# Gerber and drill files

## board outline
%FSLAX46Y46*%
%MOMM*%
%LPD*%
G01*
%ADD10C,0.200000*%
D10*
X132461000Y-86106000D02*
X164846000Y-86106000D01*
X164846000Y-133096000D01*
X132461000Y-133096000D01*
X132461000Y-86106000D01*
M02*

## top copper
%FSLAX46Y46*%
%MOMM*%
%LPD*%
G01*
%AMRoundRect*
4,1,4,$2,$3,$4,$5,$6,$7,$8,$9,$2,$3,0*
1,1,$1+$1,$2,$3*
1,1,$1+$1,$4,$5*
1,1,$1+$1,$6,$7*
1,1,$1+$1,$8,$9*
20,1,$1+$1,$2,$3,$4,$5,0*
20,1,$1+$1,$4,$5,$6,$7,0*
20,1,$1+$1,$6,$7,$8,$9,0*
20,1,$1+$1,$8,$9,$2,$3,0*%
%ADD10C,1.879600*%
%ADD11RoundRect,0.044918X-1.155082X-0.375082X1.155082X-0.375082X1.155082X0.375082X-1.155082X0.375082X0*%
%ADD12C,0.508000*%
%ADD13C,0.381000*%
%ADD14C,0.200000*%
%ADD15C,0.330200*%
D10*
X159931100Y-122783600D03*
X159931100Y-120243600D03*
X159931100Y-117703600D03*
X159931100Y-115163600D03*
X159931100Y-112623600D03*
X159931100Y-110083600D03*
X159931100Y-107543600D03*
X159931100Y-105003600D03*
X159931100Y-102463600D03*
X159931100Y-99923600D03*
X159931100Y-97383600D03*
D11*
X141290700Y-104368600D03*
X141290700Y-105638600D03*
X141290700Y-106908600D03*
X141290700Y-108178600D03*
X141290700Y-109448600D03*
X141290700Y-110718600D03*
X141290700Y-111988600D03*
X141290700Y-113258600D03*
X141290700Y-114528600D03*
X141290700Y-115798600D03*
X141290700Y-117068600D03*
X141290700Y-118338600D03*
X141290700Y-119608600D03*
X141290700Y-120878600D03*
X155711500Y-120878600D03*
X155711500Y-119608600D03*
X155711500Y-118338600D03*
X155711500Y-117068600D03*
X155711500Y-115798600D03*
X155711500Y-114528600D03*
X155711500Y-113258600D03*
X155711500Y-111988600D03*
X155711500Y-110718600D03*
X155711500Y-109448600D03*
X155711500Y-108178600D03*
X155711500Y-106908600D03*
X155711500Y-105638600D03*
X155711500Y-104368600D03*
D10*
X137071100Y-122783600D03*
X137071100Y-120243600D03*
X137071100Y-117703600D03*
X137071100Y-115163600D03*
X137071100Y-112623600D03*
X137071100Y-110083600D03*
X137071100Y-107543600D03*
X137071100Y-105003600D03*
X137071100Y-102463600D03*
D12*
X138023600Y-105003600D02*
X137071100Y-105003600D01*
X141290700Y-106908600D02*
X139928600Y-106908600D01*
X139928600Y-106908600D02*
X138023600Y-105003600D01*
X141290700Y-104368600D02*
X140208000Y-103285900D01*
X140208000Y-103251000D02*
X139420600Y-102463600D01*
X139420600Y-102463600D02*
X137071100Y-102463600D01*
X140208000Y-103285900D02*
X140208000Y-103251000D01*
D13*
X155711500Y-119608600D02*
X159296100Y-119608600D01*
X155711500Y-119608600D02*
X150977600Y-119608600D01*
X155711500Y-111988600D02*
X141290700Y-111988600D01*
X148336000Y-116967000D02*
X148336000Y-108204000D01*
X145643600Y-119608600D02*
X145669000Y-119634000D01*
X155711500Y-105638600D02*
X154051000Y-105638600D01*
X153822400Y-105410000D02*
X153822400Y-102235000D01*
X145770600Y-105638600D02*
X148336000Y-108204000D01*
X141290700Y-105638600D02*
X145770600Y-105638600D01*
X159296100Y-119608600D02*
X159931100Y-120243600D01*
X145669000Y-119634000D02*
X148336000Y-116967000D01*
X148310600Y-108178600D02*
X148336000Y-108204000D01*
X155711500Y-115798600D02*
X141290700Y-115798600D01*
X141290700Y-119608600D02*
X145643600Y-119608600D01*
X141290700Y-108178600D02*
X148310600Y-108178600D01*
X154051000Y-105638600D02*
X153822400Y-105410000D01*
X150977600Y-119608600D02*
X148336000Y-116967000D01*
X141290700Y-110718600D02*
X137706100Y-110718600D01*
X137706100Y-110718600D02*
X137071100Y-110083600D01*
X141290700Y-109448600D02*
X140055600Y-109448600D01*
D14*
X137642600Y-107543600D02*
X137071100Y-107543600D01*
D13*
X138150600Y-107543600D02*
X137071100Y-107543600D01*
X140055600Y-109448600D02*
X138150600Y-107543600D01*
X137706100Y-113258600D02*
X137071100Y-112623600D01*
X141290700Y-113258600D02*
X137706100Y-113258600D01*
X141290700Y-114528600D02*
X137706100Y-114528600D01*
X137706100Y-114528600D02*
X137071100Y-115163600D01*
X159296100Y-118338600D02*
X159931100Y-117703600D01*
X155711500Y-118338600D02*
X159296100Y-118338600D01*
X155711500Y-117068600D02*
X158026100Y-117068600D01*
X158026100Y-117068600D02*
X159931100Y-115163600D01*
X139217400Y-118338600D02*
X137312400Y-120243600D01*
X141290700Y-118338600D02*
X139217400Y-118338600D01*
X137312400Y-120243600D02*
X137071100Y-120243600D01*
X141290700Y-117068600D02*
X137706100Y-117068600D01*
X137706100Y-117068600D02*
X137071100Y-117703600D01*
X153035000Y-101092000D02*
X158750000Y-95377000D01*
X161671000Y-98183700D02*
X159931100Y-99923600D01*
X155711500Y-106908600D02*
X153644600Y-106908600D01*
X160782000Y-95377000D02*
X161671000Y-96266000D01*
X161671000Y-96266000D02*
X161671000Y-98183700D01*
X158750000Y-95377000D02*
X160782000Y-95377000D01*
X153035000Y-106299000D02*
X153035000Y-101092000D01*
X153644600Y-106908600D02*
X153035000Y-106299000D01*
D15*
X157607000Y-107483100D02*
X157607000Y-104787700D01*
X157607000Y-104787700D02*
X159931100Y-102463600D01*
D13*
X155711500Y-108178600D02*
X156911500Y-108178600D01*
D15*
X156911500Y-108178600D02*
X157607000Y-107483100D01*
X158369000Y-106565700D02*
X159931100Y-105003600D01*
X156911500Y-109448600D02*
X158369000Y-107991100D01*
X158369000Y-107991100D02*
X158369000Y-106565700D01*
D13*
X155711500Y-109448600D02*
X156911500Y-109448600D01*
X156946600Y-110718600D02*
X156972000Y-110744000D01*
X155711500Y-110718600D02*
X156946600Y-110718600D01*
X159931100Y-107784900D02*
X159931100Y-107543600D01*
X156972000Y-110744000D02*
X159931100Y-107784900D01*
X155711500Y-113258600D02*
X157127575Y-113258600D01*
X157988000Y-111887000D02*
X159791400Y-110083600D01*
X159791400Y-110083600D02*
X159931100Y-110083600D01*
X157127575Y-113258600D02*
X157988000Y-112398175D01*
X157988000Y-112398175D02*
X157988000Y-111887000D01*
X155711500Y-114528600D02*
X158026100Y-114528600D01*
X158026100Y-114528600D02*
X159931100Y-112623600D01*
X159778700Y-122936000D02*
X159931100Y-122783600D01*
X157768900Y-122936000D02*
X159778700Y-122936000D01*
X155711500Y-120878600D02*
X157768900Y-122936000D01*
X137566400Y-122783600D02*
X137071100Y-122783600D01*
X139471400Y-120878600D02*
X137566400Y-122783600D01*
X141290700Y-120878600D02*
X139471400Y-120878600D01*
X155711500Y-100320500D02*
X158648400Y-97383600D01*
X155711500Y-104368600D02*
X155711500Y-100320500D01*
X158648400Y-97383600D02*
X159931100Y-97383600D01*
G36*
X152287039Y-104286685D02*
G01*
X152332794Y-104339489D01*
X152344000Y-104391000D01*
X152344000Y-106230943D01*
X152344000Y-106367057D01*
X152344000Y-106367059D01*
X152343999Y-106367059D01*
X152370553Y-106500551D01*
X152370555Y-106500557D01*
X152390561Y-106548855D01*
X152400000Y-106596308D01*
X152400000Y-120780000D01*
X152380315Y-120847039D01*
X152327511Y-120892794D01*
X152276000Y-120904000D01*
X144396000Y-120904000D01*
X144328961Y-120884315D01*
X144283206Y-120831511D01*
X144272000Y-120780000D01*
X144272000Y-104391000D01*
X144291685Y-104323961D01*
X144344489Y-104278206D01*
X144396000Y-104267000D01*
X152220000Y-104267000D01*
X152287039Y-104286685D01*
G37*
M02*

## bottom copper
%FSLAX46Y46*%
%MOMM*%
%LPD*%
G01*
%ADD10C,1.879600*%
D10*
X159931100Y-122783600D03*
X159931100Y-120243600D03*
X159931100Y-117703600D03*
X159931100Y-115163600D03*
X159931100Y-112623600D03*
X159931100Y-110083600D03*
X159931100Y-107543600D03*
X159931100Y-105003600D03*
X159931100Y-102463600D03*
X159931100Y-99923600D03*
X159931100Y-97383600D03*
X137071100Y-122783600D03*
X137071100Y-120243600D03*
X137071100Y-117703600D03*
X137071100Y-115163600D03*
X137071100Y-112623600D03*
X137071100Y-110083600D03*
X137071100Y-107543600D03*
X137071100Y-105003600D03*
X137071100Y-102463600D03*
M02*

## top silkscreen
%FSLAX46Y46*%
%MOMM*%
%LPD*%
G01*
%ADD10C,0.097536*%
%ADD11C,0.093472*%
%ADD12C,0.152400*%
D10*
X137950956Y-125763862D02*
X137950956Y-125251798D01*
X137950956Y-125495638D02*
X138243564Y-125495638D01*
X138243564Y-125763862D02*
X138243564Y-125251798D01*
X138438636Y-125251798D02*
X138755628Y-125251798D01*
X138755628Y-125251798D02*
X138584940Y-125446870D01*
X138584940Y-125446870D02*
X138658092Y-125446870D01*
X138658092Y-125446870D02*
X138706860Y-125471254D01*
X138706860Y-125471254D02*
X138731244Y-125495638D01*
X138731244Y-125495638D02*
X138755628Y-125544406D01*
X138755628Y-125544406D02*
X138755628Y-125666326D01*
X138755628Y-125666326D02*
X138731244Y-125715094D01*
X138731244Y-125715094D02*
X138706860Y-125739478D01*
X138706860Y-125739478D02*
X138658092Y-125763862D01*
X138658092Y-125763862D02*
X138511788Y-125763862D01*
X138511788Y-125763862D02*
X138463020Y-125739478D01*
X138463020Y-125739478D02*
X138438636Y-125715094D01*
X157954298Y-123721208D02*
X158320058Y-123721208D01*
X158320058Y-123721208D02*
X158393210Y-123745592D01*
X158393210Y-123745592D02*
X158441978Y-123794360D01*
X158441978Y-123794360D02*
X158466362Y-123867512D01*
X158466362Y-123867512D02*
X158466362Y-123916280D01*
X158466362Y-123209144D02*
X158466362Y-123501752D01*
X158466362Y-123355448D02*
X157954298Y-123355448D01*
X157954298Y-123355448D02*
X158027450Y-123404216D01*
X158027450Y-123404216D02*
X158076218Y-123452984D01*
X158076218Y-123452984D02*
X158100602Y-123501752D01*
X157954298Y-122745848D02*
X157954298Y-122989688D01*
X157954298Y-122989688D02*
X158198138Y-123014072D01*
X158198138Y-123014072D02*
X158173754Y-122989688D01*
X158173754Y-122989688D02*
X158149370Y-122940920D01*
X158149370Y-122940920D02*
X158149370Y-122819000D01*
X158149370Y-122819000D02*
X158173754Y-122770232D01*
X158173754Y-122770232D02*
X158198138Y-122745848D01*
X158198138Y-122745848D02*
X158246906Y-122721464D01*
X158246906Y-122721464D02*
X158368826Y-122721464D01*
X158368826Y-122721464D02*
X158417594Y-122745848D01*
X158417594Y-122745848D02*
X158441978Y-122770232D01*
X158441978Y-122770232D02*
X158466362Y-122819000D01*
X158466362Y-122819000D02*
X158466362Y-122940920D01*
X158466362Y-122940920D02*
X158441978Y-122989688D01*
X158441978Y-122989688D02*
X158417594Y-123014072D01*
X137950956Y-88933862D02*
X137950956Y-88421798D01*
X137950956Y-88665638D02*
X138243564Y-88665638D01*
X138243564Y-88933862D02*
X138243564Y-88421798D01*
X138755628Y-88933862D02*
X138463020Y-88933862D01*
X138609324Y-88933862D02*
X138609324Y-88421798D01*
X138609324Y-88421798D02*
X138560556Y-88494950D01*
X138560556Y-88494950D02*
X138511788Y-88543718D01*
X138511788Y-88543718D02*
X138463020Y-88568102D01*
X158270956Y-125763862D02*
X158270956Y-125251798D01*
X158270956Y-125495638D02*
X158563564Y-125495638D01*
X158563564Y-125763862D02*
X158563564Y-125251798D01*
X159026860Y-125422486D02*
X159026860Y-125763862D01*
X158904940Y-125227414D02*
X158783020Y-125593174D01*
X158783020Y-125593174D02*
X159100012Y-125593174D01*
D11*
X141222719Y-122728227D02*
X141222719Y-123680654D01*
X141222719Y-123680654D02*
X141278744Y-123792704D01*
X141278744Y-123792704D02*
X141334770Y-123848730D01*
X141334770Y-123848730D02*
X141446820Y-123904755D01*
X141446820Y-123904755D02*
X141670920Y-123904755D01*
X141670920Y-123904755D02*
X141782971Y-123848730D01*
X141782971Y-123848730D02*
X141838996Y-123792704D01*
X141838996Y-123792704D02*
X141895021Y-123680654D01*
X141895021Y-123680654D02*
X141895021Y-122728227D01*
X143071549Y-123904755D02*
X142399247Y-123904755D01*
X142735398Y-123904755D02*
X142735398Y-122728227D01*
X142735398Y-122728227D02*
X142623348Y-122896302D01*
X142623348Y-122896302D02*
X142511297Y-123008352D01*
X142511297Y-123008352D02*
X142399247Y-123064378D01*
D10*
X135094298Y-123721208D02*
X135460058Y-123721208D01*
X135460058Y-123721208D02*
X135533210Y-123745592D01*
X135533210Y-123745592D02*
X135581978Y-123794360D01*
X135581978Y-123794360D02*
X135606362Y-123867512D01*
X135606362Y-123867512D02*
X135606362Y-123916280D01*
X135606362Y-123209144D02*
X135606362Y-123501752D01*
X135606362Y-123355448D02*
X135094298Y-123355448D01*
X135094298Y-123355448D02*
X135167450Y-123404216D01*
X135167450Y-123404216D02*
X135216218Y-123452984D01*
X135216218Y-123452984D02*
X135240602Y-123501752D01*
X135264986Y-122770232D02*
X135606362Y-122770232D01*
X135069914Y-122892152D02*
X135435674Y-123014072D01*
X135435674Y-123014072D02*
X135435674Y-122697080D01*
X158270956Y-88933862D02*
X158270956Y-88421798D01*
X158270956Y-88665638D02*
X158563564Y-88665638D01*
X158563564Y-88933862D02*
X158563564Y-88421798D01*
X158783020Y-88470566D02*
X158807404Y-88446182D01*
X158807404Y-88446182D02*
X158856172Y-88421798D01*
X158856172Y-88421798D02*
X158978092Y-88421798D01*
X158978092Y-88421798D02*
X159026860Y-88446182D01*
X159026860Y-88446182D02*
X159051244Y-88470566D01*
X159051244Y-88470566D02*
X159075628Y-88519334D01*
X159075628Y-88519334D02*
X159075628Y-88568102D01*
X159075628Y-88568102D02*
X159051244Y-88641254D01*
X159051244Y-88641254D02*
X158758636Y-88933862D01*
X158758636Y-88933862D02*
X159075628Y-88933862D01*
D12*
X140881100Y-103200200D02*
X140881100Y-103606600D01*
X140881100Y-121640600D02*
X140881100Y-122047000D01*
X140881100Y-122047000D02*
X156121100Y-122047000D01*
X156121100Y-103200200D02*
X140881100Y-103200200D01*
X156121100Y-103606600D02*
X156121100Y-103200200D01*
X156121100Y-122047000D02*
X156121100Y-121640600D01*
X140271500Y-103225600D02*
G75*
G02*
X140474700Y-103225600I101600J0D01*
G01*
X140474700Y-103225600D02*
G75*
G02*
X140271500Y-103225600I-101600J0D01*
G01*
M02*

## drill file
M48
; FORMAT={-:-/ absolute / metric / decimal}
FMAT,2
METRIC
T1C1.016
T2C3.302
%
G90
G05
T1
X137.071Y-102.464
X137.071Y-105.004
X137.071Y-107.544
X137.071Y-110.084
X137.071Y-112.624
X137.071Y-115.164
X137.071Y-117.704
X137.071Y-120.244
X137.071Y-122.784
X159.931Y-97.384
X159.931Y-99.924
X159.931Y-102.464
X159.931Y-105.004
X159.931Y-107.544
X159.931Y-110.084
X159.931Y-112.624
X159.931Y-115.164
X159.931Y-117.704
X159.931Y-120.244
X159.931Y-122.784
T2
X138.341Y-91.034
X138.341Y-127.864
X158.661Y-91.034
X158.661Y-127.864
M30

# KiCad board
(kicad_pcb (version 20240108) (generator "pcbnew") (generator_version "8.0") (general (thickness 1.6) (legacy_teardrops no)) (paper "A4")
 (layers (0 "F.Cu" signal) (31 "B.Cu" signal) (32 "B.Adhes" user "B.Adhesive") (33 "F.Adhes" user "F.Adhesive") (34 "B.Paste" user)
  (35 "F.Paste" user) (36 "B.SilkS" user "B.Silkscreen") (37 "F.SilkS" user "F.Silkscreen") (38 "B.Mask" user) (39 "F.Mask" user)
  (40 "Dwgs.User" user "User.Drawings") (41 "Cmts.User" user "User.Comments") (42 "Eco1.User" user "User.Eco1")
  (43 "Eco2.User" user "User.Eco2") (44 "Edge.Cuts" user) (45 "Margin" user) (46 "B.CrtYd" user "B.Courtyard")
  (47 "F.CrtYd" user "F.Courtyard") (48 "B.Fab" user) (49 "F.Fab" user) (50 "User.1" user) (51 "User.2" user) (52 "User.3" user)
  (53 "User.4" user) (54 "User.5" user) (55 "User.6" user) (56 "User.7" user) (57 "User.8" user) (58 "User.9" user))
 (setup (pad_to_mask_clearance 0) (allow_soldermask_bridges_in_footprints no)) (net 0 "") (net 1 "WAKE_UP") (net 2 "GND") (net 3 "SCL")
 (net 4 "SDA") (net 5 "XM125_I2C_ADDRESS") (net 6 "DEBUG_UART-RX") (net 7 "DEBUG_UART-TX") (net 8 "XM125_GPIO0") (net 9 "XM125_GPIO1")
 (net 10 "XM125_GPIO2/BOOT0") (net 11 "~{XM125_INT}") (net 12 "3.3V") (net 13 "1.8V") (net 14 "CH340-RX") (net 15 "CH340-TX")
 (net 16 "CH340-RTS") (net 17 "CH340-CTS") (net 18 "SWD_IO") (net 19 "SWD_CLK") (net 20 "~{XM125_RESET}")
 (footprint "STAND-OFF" (layer "F.Cu") (at 138.3411 127.8636)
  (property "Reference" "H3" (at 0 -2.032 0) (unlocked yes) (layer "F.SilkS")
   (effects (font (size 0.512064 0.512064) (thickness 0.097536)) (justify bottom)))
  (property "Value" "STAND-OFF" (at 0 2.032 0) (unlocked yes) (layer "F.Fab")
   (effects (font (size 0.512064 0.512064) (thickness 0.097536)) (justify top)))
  (pad "" np_thru_hole circle (at 0 0) (size 3.302 3.302) (drill 3.302) (layers "*.Cu" "*.Mask")))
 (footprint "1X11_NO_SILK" (layer "F.Cu") (at 159.9311 122.7836 90)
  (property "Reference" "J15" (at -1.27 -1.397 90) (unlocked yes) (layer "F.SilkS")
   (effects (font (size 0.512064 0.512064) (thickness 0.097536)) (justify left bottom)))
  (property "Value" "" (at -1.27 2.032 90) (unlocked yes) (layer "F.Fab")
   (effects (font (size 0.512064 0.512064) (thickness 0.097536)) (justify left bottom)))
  (pad "1" thru_hole circle (at 0 0 180) (size 1.8796 1.8796) (drill 1.016) (layers "*.Cu" "*.Mask") (remove_unused_layers no)
   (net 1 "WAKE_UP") (solder_mask_margin 0.0762) (thermal_bridge_angle 0))
  (pad "2" thru_hole circle (at 2.54 0 180) (size 1.8796 1.8796) (drill 1.016) (layers "*.Cu" "*.Mask") (remove_unused_layers no)
   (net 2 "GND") (solder_mask_margin 0.0762) (thermal_bridge_angle 0))
  (pad "3" thru_hole circle (at 5.08 0 180) (size 1.8796 1.8796) (drill 1.016) (layers "*.Cu" "*.Mask") (remove_unused_layers no)
   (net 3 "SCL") (solder_mask_margin 0.0762) (thermal_bridge_angle 0))
  (pad "4" thru_hole circle (at 7.62 0 180) (size 1.8796 1.8796) (drill 1.016) (layers "*.Cu" "*.Mask") (remove_unused_layers no)
   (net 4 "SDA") (solder_mask_margin 0.0762) (thermal_bridge_angle 0))
  (pad "5" thru_hole circle (at 10.16 0 180) (size 1.8796 1.8796) (drill 1.016) (layers "*.Cu" "*.Mask") (remove_unused_layers no)
   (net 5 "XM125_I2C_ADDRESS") (solder_mask_margin 0.0762) (thermal_bridge_angle 0))
  (pad "6" thru_hole circle (at 12.7 0 180) (size 1.8796 1.8796) (drill 1.016) (layers "*.Cu" "*.Mask") (remove_unused_layers no)
   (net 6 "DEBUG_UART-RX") (solder_mask_margin 0.0762) (thermal_bridge_angle 0))
  (pad "7" thru_hole circle (at 15.24 0 180) (size 1.8796 1.8796) (drill 1.016) (layers "*.Cu" "*.Mask") (remove_unused_layers no)
   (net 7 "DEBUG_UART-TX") (solder_mask_margin 0.0762) (thermal_bridge_angle 0))
  (pad "8" thru_hole circle (at 17.78 0 180) (size 1.8796 1.8796) (drill 1.016) (layers "*.Cu" "*.Mask") (remove_unused_layers no)
   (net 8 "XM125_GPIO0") (solder_mask_margin 0.0762) (thermal_bridge_angle 0))
  (pad "9" thru_hole circle (at 20.32 0 180) (size 1.8796 1.8796) (drill 1.016) (layers "*.Cu" "*.Mask") (remove_unused_layers no)
   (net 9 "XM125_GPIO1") (solder_mask_margin 0.0762) (thermal_bridge_angle 0))
  (pad "10" thru_hole circle (at 22.86 0 180) (size 1.8796 1.8796) (drill 1.016) (layers "*.Cu" "*.Mask") (remove_unused_layers no)
   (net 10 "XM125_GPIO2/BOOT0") (solder_mask_margin 0.0762) (thermal_bridge_angle 0))
  (pad "11" thru_hole circle (at 25.4 0 180) (size 1.8796 1.8796) (drill 1.016) (layers "*.Cu" "*.Mask") (remove_unused_layers no)
   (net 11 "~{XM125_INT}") (solder_mask_margin 0.0762) (thermal_bridge_angle 0)))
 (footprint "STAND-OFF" (layer "F.Cu") (at 138.3411 91.0336)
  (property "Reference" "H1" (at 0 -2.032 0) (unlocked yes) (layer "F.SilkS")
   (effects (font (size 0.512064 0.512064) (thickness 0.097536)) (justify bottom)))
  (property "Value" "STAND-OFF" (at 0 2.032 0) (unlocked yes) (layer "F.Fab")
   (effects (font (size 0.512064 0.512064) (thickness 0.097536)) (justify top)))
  (pad "" np_thru_hole circle (at 0 0) (size 3.302 3.302) (drill 3.302) (layers "*.Cu" "*.Mask")))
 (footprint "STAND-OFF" (layer "F.Cu") (at 158.6611 127.8636)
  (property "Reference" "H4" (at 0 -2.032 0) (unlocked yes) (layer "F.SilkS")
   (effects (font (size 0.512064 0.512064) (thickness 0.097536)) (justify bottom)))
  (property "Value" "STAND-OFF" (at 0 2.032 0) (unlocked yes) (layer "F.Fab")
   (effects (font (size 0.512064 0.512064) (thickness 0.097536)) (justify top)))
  (pad "" np_thru_hole circle (at 0 0) (size 3.302 3.302) (drill 3.302) (layers "*.Cu" "*.Mask")))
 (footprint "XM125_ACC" (layer "F.Cu") (at 148.5011 112.6236)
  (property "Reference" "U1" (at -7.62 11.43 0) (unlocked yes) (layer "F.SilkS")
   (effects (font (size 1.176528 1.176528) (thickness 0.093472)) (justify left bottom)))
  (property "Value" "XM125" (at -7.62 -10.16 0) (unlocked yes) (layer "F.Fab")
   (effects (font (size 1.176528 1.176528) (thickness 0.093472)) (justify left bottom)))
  (fp_line (start -7.62 -9.4234) (end -7.62 -9.017) (stroke (width 0.1524) (type solid)) (layer "F.SilkS"))
  (fp_line (start -7.62 9.017) (end -7.62 9.4234) (stroke (width 0.1524) (type solid)) (layer "F.SilkS"))
  (fp_line (start -7.62 9.4234) (end 7.62 9.4234) (stroke (width 0.1524) (type solid)) (layer "F.SilkS"))
  (fp_line (start 7.62 -9.4234) (end -7.62 -9.4234) (stroke (width 0.1524) (type solid)) (layer "F.SilkS"))
  (fp_line (start 7.62 -9.017) (end 7.62 -9.4234) (stroke (width 0.1524) (type solid)) (layer "F.SilkS"))
  (fp_line (start 7.62 9.4234) (end 7.62 9.017) (stroke (width 0.1524) (type solid)) (layer "F.SilkS"))
  (fp_arc (start -8.2296 -9.398) (mid -8.128 -9.4996) (end -8.0264 -9.398) (stroke (width 0.1524) (type solid)) (layer "F.SilkS"))
  (fp_arc (start -8.0264 -9.398) (mid -8.128 -9.2964) (end -8.2296 -9.398) (stroke (width 0.1524) (type solid)) (layer "F.SilkS"))
  (pad "1" smd roundrect (at -7.2104 -8.255) (size 2.4 0.84) (layers "F.Cu" "F.Paste" "F.Mask") (roundrect_rratio 0.05347368421)
   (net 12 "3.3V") (solder_mask_margin 0.0762) (thermal_bridge_angle 0))
  (pad "2" smd roundrect (at -7.2104 -6.985) (size 2.4 0.84) (layers "F.Cu" "F.Paste" "F.Mask") (roundrect_rratio 0.05347368421)
   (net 2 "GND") (solder_mask_margin 0.0762) (thermal_bridge_angle 0))
  (pad "3" smd roundrect (at -7.2104 -5.715) (size 2.4 0.84) (layers "F.Cu" "F.Paste" "F.Mask") (roundrect_rratio 0.05347368421)
   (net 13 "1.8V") (solder_mask_margin 0.0762) (thermal_bridge_angle 0))
  (pad "4" smd roundrect (at -7.2104 -4.445) (size 2.4 0.84) (layers "F.Cu" "F.Paste" "F.Mask") (roundrect_rratio 0.05347368421)
   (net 2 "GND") (solder_mask_margin 0.0762) (thermal_bridge_angle 0))
  (pad "5" smd roundrect (at -7.2104 -3.175) (size 2.4 0.84) (layers "F.Cu" "F.Paste" "F.Mask") (roundrect_rratio 0.05347368421)
   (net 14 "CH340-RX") (solder_mask_margin 0.0762) (thermal_bridge_angle 0))
  (pad "6" smd roundrect (at -7.2104 -1.905) (size 2.4 0.84) (layers "F.Cu" "F.Paste" "F.Mask") (roundrect_rratio 0.05347368421)
   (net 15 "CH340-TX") (solder_mask_margin 0.0762) (thermal_bridge_angle 0))
  (pad "7" smd roundrect (at -7.2104 -0.635) (size 2.4 0.84) (layers "F.Cu" "F.Paste" "F.Mask") (roundrect_rratio 0.05347368421)
   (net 2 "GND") (solder_mask_margin 0.0762) (thermal_bridge_angle 0))
  (pad "8" smd roundrect (at -7.2104 0.635) (size 2.4 0.84) (layers "F.Cu" "F.Paste" "F.Mask") (roundrect_rratio 0.05347368421)
   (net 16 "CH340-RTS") (solder_mask_margin 0.0762) (thermal_bridge_angle 0))
  (pad "9" smd roundrect (at -7.2104 1.905) (size 2.4 0.84) (layers "F.Cu" "F.Paste" "F.Mask") (roundrect_rratio 0.05347368421)
   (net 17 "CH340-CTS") (solder_mask_margin 0.0762) (thermal_bridge_angle 0))
  (pad "10" smd roundrect (at -7.2104 3.175) (size 2.4 0.84) (layers "F.Cu" "F.Paste" "F.Mask") (roundrect_rratio 0.05347368421)
   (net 2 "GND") (solder_mask_margin 0.0762) (thermal_bridge_angle 0))
  (pad "11" smd roundrect (at -7.2104 4.445) (size 2.4 0.84) (layers "F.Cu" "F.Paste" "F.Mask") (roundrect_rratio 0.05347368421)
   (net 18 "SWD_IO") (solder_mask_margin 0.0762) (thermal_bridge_angle 0))
  (pad "12" smd roundrect (at -7.2104 5.715) (size 2.4 0.84) (layers "F.Cu" "F.Paste" "F.Mask") (roundrect_rratio 0.05347368421)
   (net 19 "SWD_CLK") (solder_mask_margin 0.0762) (thermal_bridge_angle 0))
  (pad "13" smd roundrect (at -7.2104 6.985) (size 2.4 0.84) (layers "F.Cu" "F.Paste" "F.Mask") (roundrect_rratio 0.05347368421)
   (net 2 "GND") (solder_mask_margin 0.0762) (thermal_bridge_angle 0))
  (pad "14" smd roundrect (at -7.2104 8.255) (size 2.4 0.84) (layers "F.Cu" "F.Paste" "F.Mask") (roundrect_rratio 0.05347368421)
   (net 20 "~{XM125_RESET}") (solder_mask_margin 0.0762) (thermal_bridge_angle 0))
  (pad "15" smd roundrect (at 7.2104 8.255) (size 2.4 0.84) (layers "F.Cu" "F.Paste" "F.Mask") (roundrect_rratio 0.05347368421)
   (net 1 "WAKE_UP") (solder_mask_margin 0.0762) (thermal_bridge_angle 0))
  (pad "16" smd roundrect (at 7.2104 6.985) (size 2.4 0.84) (layers "F.Cu" "F.Paste" "F.Mask") (roundrect_rratio 0.05347368421)
   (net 2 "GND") (solder_mask_margin 0.0762) (thermal_bridge_angle 0))
  (pad "17" smd roundrect (at 7.2104 5.715) (size 2.4 0.84) (layers "F.Cu" "F.Paste" "F.Mask") (roundrect_rratio 0.05347368421)
   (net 3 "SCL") (solder_mask_margin 0.0762) (thermal_bridge_angle 0))
  (pad "18" smd roundrect (at 7.2104 4.445) (size 2.4 0.84) (layers "F.Cu" "F.Paste" "F.Mask") (roundrect_rratio 0.05347368421)
   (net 4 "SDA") (solder_mask_margin 0.0762) (thermal_bridge_angle 0))
  (pad "19" smd roundrect (at 7.2104 3.175) (size 2.4 0.84) (layers "F.Cu" "F.Paste" "F.Mask") (roundrect_rratio 0.05347368421)
   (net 2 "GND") (solder_mask_margin 0.0762) (thermal_bridge_angle 0))
  (pad "20" smd roundrect (at 7.2104 1.905) (size 2.4 0.84) (layers "F.Cu" "F.Paste" "F.Mask") (roundrect_rratio 0.05347368421)
   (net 5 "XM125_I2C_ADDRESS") (solder_mask_margin 0.0762) (thermal_bridge_angle 0))
  (pad "21" smd roundrect (at 7.2104 0.635) (size 2.4 0.84) (layers "F.Cu" "F.Paste" "F.Mask") (roundrect_rratio 0.05347368421)
   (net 6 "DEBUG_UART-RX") (solder_mask_margin 0.0762) (thermal_bridge_angle 0))
  (pad "22" smd roundrect (at 7.2104 -0.635) (size 2.4 0.84) (layers "F.Cu" "F.Paste" "F.Mask") (roundrect_rratio 0.05347368421)
   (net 2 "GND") (solder_mask_margin 0.0762) (thermal_bridge_angle 0))
  (pad "23" smd roundrect (at 7.2104 -1.905) (size 2.4 0.84) (layers "F.Cu" "F.Paste" "F.Mask") (roundrect_rratio 0.05347368421)
   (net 7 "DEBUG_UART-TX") (solder_mask_margin 0.0762) (thermal_bridge_angle 0))
  (pad "24" smd roundrect (at 7.2104 -3.175) (size 2.4 0.84) (layers "F.Cu" "F.Paste" "F.Mask") (roundrect_rratio 0.05347368421)
   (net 8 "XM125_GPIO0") (solder_mask_margin 0.0762) (thermal_bridge_angle 0))
  (pad "25" smd roundrect (at 7.2104 -4.445) (size 2.4 0.84) (layers "F.Cu" "F.Paste" "F.Mask") (roundrect_rratio 0.05347368421)
   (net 9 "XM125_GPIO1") (solder_mask_margin 0.0762) (thermal_bridge_angle 0))
  (pad "26" smd roundrect (at 7.2104 -5.715) (size 2.4 0.84) (layers "F.Cu" "F.Paste" "F.Mask") (roundrect_rratio 0.05347368421)
   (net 10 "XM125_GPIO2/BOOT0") (solder_mask_margin 0.0762) (thermal_bridge_angle 0))
  (pad "27" smd roundrect (at 7.2104 -6.985) (size 2.4 0.84) (layers "F.Cu" "F.Paste" "F.Mask") (roundrect_rratio 0.05347368421)
   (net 2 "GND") (solder_mask_margin 0.0762) (thermal_bridge_angle 0))
  (pad "28" smd roundrect (at 7.2104 -8.255) (size 2.4 0.84) (layers "F.Cu" "F.Paste" "F.Mask") (roundrect_rratio 0.05347368421)
   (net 11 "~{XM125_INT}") (solder_mask_margin 0.0762) (thermal_bridge_angle 0)))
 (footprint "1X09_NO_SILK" (layer "F.Cu") (at 137.0711 122.7836 90)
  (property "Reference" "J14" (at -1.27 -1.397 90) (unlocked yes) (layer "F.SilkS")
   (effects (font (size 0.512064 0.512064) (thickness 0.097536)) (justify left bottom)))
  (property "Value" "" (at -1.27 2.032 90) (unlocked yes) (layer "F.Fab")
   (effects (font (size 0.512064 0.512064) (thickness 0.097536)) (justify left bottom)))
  (pad "1" thru_hole circle (at 0 0 180) (size 1.8796 1.8796) (drill 1.016) (layers "*.Cu" "*.Mask") (remove_unused_layers no)
   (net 20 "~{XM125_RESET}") (solder_mask_margin 0.0762) (thermal_bridge_angle 0))
  (pad "2" thru_hole circle (at 2.54 0 180) (size 1.8796 1.8796) (drill 1.016) (layers "*.Cu" "*.Mask") (remove_unused_layers no)
   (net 19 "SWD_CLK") (solder_mask_margin 0.0762) (thermal_bridge_angle 0))
  (pad "3" thru_hole circle (at 5.08 0 180) (size 1.8796 1.8796) (drill 1.016) (layers "*.Cu" "*.Mask") (remove_unused_layers no)
   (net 18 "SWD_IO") (solder_mask_margin 0.0762) (thermal_bridge_angle 0))
  (pad "4" thru_hole circle (at 7.62 0 180) (size 1.8796 1.8796) (drill 1.016) (layers "*.Cu" "*.Mask") (remove_unused_layers no)
   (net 17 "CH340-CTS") (solder_mask_margin 0.0762) (thermal_bridge_angle 0))
  (pad "5" thru_hole circle (at 10.16 0 180) (size 1.8796 1.8796) (drill 1.016) (layers "*.Cu" "*.Mask") (remove_unused_layers no)
   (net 16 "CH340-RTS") (solder_mask_margin 0.0762) (thermal_bridge_angle 0))
  (pad "6" thru_hole circle (at 12.7 0 180) (size 1.8796 1.8796) (drill 1.016) (layers "*.Cu" "*.Mask") (remove_unused_layers no)
   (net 15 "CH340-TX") (solder_mask_margin 0.0762) (thermal_bridge_angle 0))
  (pad "7" thru_hole circle (at 15.24 0 180) (size 1.8796 1.8796) (drill 1.016) (layers "*.Cu" "*.Mask") (remove_unused_layers no)
   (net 14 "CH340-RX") (solder_mask_margin 0.0762) (thermal_bridge_angle 0))
  (pad "8" thru_hole circle (at 17.78 0 180) (size 1.8796 1.8796) (drill 1.016) (layers "*.Cu" "*.Mask") (remove_unused_layers no)
   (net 13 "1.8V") (solder_mask_margin 0.0762) (thermal_bridge_angle 0))
  (pad "9" thru_hole circle (at 20.32 0 180) (size 1.8796 1.8796) (drill 1.016) (layers "*.Cu" "*.Mask") (remove_unused_layers no)
   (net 12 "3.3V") (solder_mask_margin 0.0762) (thermal_bridge_angle 0)))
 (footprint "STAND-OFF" (layer "F.Cu") (at 158.6611 91.0336)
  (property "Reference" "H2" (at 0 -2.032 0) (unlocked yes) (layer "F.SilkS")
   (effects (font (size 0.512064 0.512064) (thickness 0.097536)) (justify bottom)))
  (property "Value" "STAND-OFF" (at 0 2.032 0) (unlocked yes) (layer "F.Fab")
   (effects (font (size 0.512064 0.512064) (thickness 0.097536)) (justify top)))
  (pad "" np_thru_hole circle (at 0 0) (size 3.302 3.302) (drill 3.302) (layers "*.Cu" "*.Mask")))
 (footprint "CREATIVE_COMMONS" (layer "F.Cu") (at 120.5611 165.9636)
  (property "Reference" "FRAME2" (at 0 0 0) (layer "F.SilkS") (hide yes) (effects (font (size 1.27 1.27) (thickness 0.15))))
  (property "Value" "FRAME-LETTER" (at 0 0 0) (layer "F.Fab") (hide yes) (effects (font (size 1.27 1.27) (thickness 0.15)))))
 (gr_rect (start 132.461 86.106) (end 164.846 133.096) (stroke (width 0.2) (type default)) (fill none) (layer "Edge.Cuts"))
 (segment (start 138.0236 105.0036) (end 137.0711 105.0036) (width 0.508) (layer "F.Cu") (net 13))
 (segment (start 141.2907 106.9086) (end 139.9286 106.9086) (width 0.508) (layer "F.Cu") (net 13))
 (segment (start 139.9286 106.9086) (end 138.0236 105.0036) (width 0.508) (layer "F.Cu") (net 13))
 (segment (start 141.2907 104.3686) (end 140.208 103.2859) (width 0.508) (layer "F.Cu") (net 12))
 (segment (start 140.208 103.251) (end 139.4206 102.4636) (width 0.508) (layer "F.Cu") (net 12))
 (segment (start 139.4206 102.4636) (end 137.0711 102.4636) (width 0.508) (layer "F.Cu") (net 12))
 (segment (start 140.208 103.2859) (end 140.208 103.251) (width 0.508) (layer "F.Cu") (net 12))
 (segment (start 155.7115 119.6086) (end 159.2961 119.6086) (width 0.381) (layer "F.Cu") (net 2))
 (segment (start 155.7115 119.6086) (end 150.9776 119.6086) (width 0.381) (layer "F.Cu") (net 2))
 (segment (start 155.7115 111.9886) (end 141.2907 111.9886) (width 0.381) (layer "F.Cu") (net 2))
 (segment (start 148.336 116.967) (end 148.336 108.204) (width 0.381) (layer "F.Cu") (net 2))
 (segment (start 145.6436 119.6086) (end 145.669 119.634) (width 0.381) (layer "F.Cu") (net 2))
 (segment (start 155.7115 105.6386) (end 154.051 105.6386) (width 0.381) (layer "F.Cu") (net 2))
 (segment (start 153.8224 105.41) (end 153.8224 102.235) (width 0.381) (layer "F.Cu") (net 2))
 (segment (start 145.7706 105.6386) (end 148.336 108.204) (width 0.381) (layer "F.Cu") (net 2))
 (segment (start 141.2907 105.6386) (end 145.7706 105.6386) (width 0.381) (layer "F.Cu") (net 2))
 (segment (start 159.2961 119.6086) (end 159.9311 120.2436) (width 0.381) (layer "F.Cu") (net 2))
 (segment (start 145.669 119.634) (end 148.336 116.967) (width 0.381) (layer "F.Cu") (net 2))
 (segment (start 148.3106 108.1786) (end 148.336 108.204) (width 0.381) (layer "F.Cu") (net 2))
 (segment (start 155.7115 115.7986) (end 141.2907 115.7986) (width 0.381) (layer "F.Cu") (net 2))
 (segment (start 141.2907 119.6086) (end 145.6436 119.6086) (width 0.381) (layer "F.Cu") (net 2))
 (segment (start 141.2907 108.1786) (end 148.3106 108.1786) (width 0.381) (layer "F.Cu") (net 2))
 (segment (start 154.051 105.6386) (end 153.8224 105.41) (width 0.381) (layer "F.Cu") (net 2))
 (segment (start 150.9776 119.6086) (end 148.336 116.967) (width 0.381) (layer "F.Cu") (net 2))
 (segment (start 141.2907 110.7186) (end 137.7061 110.7186) (width 0.381) (layer "F.Cu") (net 15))
 (segment (start 137.7061 110.7186) (end 137.0711 110.0836) (width 0.381) (layer "F.Cu") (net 15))
 (segment (start 141.2907 109.4486) (end 140.0556 109.4486) (width 0.381) (layer "F.Cu") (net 14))
 (segment (start 137.6426 107.5436) (end 137.0711 107.5436) (width 0.2) (layer "F.Cu") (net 14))
 (segment (start 138.1506 107.5436) (end 137.0711 107.5436) (width 0.381) (layer "F.Cu") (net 14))
 (segment (start 140.0556 109.4486) (end 138.1506 107.5436) (width 0.381) (layer "F.Cu") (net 14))
 (segment (start 137.7061 113.2586) (end 137.0711 112.6236) (width 0.381) (layer "F.Cu") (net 16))
 (segment (start 141.2907 113.2586) (end 137.7061 113.2586) (width 0.381) (layer "F.Cu") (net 16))
 (segment (start 141.2907 114.5286) (end 137.7061 114.5286) (width 0.381) (layer "F.Cu") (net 17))
 (segment (start 137.7061 114.5286) (end 137.0711 115.1636) (width 0.381) (layer "F.Cu") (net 17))
 (segment (start 159.2961 118.3386) (end 159.9311 117.7036) (width 0.381) (layer "F.Cu") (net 3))
 (segment (start 155.7115 118.3386) (end 159.2961 118.3386) (width 0.381) (layer "F.Cu") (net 3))
 (segment (start 155.7115 117.0686) (end 158.0261 117.0686) (width 0.381) (layer "F.Cu") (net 4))
 (segment (start 158.0261 117.0686) (end 159.9311 115.1636) (width 0.381) (layer "F.Cu") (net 4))
 (segment (start 139.2174 118.3386) (end 137.3124 120.2436) (width 0.381) (layer "F.Cu") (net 19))
 (segment (start 141.2907 118.3386) (end 139.2174 118.3386) (width 0.381) (layer "F.Cu") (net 19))
 (segment (start 137.3124 120.2436) (end 137.0711 120.2436) (width 0.381) (layer "F.Cu") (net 19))
 (segment (start 141.2907 117.0686) (end 137.7061 117.0686) (width 0.381) (layer "F.Cu") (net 18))
 (segment (start 137.7061 117.0686) (end 137.0711 117.7036) (width 0.381) (layer "F.Cu") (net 18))
 (segment (start 153.035 101.092) (end 158.75 95.377) (width 0.381) (layer "F.Cu") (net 10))
 (segment (start 161.671 98.1837) (end 159.9311 99.9236) (width 0.381) (layer "F.Cu") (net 10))
 (segment (start 155.7115 106.9086) (end 153.6446 106.9086) (width 0.381) (layer "F.Cu") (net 10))
 (segment (start 160.782 95.377) (end 161.671 96.266) (width 0.381) (layer "F.Cu") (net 10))
 (segment (start 161.671 96.266) (end 161.671 98.1837) (width 0.381) (layer "F.Cu") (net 10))
 (segment (start 158.75 95.377) (end 160.782 95.377) (width 0.381) (layer "F.Cu") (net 10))
 (segment (start 153.035 106.299) (end 153.035 101.092) (width 0.381) (layer "F.Cu") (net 10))
 (segment (start 153.6446 106.9086) (end 153.035 106.299) (width 0.381) (layer "F.Cu") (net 10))
 (segment (start 157.607 107.4831) (end 157.607 104.7877) (width 0.3302) (layer "F.Cu") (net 9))
 (segment (start 157.607 104.7877) (end 159.9311 102.4636) (width 0.3302) (layer "F.Cu") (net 9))
 (segment (start 155.7115 108.1786) (end 156.9115 108.1786) (width 0.381) (layer "F.Cu") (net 9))
 (segment (start 156.9115 108.1786) (end 157.607 107.4831) (width 0.3302) (layer "F.Cu") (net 9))
 (segment (start 158.369 106.5657) (end 159.9311 105.0036) (width 0.3302) (layer "F.Cu") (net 8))
 (segment (start 156.9115 109.4486) (end 158.369 107.9911) (width 0.3302) (layer "F.Cu") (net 8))
 (segment (start 158.369 107.9911) (end 158.369 106.5657) (width 0.3302) (layer "F.Cu") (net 8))
 (segment (start 155.7115 109.4486) (end 156.9115 109.4486) (width 0.381) (layer "F.Cu") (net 8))
 (segment (start 156.9466 110.7186) (end 156.972 110.744) (width 0.381) (layer "F.Cu") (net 7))
 (segment (start 155.7115 110.7186) (end 156.9466 110.7186) (width 0.381) (layer "F.Cu") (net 7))
 (segment (start 159.9311 107.7849) (end 159.9311 107.5436) (width 0.381) (layer "F.Cu") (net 7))
 (segment (start 156.972 110.744) (end 159.9311 107.7849) (width 0.381) (layer "F.Cu") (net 7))
 (segment (start 155.7115 113.2586) (end 157.127575 113.2586) (width 0.381) (layer "F.Cu") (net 6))
 (segment (start 157.988 111.887) (end 159.7914 110.0836) (width 0.381) (layer "F.Cu") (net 6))
 (segment (start 159.7914 110.0836) (end 159.9311 110.0836) (width 0.381) (layer "F.Cu") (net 6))
 (segment (start 157.127575 113.2586) (end 157.988 112.398175) (width 0.381) (layer "F.Cu") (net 6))
 (segment (start 157.988 112.398175) (end 157.988 111.887) (width 0.381) (layer "F.Cu") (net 6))
 (segment (start 155.7115 114.5286) (end 158.0261 114.5286) (width 0.381) (layer "F.Cu") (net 5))
 (segment (start 158.0261 114.5286) (end 159.9311 112.6236) (width 0.381) (layer "F.Cu") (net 5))
 (segment (start 159.7787 122.936) (end 159.9311 122.7836) (width 0.381) (layer "F.Cu") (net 1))
 (segment (start 157.7689 122.936) (end 159.7787 122.936) (width 0.381) (layer "F.Cu") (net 1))
 (segment (start 155.7115 120.8786) (end 157.7689 122.936) (width 0.381) (layer "F.Cu") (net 1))
 (segment (start 137.5664 122.7836) (end 137.0711 122.7836) (width 0.381) (layer "F.Cu") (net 20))
 (segment (start 139.4714 120.8786) (end 137.5664 122.7836) (width 0.381) (layer "F.Cu") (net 20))
 (segment (start 141.2907 120.8786) (end 139.4714 120.8786) (width 0.381) (layer "F.Cu") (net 20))
 (segment (start 155.7115 100.3205) (end 158.6484 97.3836) (width 0.381) (layer "F.Cu") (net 11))
 (segment (start 155.7115 104.3686) (end 155.7115 100.3205) (width 0.381) (layer "F.Cu") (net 11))
 (segment (start 158.6484 97.3836) (end 159.9311 97.3836) (width 0.381) (layer "F.Cu") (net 11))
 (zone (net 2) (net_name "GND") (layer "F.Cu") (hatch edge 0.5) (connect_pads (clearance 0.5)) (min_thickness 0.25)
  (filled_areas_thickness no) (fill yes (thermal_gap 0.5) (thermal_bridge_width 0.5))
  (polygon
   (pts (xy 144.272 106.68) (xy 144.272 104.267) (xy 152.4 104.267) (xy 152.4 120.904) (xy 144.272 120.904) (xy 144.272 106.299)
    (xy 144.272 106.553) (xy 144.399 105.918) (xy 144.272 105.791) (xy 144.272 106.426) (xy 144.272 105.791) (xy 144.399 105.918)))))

